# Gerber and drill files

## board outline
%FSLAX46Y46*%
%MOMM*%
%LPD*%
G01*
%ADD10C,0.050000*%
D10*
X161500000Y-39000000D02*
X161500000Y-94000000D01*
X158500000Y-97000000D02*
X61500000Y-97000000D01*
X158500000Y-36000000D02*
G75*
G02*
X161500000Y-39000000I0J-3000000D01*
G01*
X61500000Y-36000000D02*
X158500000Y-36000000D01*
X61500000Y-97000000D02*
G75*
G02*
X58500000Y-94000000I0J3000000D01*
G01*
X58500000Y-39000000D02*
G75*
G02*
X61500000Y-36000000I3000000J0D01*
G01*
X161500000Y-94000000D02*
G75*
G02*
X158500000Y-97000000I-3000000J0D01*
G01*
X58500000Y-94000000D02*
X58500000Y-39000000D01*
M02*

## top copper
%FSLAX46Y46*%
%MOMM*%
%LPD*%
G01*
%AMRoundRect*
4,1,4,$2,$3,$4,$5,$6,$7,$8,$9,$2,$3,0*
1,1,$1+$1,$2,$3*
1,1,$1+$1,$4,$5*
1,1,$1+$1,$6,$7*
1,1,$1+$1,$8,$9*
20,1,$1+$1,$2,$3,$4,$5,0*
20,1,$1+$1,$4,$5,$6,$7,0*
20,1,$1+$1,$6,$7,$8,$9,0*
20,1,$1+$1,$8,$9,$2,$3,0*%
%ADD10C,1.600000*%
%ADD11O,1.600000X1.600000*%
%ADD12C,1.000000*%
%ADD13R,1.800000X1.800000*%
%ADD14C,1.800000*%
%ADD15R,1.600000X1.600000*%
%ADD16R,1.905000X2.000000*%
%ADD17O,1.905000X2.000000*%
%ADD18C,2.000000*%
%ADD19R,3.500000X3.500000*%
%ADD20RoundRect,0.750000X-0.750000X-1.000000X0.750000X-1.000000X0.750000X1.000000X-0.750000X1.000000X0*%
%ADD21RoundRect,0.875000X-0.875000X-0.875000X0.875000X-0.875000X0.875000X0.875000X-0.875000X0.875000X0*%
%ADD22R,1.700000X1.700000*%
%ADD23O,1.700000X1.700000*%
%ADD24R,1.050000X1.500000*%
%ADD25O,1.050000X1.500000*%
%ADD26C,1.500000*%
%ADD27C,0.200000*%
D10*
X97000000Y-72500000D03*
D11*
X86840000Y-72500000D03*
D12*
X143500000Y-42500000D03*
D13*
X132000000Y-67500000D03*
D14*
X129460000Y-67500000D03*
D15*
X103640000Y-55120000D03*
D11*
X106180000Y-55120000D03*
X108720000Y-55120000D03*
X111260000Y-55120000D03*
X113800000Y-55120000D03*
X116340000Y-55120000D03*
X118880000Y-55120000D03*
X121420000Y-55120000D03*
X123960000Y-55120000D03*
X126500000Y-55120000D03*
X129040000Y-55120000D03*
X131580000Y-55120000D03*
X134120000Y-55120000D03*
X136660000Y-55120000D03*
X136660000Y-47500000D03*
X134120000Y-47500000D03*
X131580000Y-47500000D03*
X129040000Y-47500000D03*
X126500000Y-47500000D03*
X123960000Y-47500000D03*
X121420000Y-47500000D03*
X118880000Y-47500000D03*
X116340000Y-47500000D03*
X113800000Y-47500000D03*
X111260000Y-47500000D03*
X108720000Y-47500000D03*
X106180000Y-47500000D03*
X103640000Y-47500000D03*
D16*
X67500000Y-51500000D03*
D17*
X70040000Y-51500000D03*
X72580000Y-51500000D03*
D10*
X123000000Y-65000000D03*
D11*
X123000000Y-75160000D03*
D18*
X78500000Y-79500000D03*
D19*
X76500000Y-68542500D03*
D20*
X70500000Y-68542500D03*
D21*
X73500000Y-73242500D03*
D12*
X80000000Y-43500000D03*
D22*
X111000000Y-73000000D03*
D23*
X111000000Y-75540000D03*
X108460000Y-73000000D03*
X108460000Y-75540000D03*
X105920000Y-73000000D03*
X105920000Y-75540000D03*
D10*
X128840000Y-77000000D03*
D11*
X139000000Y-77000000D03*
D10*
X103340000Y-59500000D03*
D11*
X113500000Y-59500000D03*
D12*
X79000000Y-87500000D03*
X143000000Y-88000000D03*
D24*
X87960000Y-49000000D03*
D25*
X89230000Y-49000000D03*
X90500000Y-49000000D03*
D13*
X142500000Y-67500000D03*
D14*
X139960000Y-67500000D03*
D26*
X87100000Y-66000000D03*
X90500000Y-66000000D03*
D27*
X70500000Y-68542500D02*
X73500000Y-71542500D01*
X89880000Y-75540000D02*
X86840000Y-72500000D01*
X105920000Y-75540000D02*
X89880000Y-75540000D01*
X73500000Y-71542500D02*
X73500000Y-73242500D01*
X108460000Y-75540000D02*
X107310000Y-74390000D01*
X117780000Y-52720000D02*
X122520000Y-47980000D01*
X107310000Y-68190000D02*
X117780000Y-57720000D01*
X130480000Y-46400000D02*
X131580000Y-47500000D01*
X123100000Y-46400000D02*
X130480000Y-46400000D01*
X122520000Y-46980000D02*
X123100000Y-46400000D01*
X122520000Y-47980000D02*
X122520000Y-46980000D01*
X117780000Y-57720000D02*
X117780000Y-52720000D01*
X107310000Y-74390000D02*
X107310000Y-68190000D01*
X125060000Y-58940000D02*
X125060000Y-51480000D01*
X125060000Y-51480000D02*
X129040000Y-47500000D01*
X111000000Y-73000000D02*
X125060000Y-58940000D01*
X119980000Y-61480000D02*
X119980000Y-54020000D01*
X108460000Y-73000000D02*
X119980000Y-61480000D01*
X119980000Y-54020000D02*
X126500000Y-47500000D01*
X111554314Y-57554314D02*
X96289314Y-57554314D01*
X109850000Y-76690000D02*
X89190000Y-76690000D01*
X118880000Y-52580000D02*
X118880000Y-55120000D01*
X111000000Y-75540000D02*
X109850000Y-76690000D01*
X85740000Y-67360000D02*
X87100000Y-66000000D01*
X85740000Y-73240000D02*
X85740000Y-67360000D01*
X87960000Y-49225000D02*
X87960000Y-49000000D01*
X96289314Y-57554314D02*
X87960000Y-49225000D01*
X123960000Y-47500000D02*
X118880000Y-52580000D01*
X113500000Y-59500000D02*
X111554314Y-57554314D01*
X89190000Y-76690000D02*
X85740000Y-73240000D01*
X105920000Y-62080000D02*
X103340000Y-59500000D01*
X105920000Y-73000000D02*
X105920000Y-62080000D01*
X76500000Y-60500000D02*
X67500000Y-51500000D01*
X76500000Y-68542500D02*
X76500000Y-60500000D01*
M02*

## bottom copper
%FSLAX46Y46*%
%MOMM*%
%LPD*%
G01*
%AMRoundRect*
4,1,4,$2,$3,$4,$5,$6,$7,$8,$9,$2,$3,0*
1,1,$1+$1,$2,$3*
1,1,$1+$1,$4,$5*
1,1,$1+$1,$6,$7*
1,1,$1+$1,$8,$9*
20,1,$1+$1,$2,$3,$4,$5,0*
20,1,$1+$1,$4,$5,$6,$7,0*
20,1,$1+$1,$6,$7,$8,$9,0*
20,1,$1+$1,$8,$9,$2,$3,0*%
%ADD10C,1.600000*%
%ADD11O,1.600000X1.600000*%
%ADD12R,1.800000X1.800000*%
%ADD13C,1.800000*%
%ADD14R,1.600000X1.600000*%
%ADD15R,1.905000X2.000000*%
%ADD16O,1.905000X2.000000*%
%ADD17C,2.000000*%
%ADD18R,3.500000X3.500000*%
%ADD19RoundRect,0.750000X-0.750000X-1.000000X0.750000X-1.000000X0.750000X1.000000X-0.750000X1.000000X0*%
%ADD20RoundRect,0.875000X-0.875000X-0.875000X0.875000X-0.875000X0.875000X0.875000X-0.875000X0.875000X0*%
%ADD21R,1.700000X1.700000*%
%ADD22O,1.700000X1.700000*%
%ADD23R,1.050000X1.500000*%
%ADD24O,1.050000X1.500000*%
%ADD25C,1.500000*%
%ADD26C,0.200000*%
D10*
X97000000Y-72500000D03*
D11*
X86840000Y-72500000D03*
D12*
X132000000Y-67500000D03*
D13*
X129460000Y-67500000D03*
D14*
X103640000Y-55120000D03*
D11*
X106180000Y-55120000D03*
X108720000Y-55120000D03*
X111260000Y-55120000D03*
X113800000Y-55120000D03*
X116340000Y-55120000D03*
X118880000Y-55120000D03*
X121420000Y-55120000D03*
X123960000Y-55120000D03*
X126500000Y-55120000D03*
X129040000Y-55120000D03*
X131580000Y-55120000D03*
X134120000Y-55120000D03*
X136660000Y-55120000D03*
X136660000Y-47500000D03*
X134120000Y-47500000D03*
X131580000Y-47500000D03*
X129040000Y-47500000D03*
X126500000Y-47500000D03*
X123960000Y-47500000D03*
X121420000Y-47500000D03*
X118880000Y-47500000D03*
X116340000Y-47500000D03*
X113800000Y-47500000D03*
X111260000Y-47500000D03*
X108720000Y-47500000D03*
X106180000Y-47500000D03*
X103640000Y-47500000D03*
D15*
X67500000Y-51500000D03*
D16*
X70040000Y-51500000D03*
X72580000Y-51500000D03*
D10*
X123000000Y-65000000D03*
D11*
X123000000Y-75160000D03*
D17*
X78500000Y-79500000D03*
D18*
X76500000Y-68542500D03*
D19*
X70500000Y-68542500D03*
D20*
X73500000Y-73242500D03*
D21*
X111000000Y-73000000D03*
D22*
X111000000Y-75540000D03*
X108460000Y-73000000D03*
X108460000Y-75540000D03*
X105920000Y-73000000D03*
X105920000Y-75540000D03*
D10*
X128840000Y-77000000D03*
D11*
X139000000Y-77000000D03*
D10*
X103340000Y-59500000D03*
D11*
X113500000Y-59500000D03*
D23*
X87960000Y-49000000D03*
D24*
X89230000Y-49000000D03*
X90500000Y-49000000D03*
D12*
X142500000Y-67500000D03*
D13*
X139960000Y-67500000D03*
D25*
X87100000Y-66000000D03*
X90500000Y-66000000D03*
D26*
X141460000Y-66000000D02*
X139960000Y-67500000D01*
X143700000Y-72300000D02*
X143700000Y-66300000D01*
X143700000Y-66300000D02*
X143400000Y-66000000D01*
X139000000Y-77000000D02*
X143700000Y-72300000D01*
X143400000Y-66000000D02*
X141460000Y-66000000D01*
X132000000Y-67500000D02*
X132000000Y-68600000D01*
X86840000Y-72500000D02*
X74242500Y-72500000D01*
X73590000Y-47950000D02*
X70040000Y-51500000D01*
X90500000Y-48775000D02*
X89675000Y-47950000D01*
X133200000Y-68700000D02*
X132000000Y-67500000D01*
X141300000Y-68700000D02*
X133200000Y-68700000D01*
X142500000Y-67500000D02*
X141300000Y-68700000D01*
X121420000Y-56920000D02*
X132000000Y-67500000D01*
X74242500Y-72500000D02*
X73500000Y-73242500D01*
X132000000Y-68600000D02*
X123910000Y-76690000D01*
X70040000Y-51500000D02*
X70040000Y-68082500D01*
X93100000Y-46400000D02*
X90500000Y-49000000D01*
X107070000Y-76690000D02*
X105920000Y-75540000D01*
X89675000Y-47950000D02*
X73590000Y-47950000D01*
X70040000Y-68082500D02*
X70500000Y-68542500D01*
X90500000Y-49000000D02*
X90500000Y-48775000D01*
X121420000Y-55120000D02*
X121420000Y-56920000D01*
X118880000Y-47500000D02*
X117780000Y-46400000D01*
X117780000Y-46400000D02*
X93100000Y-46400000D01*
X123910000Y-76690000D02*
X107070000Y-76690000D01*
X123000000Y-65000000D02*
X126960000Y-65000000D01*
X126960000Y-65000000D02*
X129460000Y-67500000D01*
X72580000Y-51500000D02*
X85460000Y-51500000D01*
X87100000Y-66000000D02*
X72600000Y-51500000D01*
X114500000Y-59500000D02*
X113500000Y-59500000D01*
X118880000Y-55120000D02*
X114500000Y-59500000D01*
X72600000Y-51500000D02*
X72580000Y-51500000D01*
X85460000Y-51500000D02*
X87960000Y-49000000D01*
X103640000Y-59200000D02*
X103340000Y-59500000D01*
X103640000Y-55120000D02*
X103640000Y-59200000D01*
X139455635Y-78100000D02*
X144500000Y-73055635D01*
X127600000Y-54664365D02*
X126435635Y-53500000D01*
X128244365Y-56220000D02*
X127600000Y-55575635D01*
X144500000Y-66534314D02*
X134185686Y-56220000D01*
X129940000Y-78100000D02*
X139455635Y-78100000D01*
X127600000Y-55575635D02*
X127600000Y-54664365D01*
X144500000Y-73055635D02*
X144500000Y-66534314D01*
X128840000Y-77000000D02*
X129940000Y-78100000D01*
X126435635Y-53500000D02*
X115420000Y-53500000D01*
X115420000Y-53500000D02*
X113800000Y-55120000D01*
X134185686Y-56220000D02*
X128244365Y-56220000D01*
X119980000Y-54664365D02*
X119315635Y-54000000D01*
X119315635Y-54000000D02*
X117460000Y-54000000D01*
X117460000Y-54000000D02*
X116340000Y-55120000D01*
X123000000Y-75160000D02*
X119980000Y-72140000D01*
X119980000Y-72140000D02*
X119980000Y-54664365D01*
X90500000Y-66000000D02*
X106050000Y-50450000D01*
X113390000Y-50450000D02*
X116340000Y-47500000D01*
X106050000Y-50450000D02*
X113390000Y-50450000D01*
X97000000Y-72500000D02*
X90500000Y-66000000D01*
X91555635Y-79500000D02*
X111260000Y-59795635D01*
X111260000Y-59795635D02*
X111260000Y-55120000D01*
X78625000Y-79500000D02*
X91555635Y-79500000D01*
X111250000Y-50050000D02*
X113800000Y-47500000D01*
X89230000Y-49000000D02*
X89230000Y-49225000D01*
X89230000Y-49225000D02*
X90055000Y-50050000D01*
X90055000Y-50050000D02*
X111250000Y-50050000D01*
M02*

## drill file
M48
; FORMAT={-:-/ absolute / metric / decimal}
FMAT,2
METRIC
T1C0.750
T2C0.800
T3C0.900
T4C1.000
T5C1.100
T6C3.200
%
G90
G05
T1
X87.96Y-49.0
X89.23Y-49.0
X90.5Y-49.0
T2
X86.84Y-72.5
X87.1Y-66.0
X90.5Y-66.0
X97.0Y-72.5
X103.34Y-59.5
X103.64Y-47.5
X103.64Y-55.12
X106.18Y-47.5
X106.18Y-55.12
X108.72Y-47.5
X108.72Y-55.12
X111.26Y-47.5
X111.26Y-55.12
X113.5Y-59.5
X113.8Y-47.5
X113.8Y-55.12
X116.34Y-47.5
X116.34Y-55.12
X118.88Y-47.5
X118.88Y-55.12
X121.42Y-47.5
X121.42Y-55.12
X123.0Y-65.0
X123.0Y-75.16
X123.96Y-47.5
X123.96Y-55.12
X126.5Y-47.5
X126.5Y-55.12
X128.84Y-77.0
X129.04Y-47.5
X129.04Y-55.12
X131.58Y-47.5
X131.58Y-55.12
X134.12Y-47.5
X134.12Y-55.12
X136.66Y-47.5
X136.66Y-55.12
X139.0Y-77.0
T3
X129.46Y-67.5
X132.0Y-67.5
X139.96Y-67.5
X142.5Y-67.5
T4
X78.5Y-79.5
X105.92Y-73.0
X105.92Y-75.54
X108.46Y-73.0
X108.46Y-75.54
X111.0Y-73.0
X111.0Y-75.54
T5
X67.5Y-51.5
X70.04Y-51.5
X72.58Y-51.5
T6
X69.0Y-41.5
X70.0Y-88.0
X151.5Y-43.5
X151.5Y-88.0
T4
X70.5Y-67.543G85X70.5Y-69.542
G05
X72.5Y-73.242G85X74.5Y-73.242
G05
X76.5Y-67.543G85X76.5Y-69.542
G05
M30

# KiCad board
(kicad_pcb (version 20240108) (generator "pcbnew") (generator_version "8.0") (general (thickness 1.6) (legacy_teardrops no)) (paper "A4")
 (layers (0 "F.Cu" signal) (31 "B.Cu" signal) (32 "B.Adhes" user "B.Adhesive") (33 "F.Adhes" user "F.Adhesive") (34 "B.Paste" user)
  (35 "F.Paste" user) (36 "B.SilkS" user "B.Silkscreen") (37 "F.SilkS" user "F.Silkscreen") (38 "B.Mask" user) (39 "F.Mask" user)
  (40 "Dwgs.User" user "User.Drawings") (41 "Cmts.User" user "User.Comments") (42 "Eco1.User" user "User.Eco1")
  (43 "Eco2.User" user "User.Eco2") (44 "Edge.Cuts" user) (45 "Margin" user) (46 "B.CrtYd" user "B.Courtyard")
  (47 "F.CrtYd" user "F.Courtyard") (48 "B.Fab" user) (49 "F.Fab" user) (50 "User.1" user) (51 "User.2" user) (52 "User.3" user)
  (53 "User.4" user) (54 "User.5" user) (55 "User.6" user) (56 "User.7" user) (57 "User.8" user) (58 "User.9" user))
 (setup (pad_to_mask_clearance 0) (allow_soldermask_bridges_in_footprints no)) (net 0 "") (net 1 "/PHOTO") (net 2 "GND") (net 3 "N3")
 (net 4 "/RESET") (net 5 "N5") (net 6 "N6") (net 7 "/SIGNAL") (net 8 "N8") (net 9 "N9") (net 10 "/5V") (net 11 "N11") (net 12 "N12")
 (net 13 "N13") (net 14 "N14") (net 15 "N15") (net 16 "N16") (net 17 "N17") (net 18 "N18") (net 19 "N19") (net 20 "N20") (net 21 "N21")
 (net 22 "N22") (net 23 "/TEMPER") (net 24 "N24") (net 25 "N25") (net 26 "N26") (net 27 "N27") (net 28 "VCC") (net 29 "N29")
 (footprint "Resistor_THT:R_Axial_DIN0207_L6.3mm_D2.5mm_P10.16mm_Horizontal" (layer "F.Cu") (at 97 72.5 180)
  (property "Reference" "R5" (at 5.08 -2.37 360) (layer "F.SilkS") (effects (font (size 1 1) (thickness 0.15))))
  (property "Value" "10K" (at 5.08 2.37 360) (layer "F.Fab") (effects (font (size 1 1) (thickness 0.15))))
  (pad "1" thru_hole circle (at 0 0 180) (size 1.6 1.6) (drill 0.8) (layers "*.Cu" "*.Mask") (remove_unused_layers no) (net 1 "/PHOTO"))
  (pad "2" thru_hole oval (at 10.16 0 180) (size 1.6 1.6) (drill 0.8) (layers "*.Cu" "*.Mask") (remove_unused_layers no) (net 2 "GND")))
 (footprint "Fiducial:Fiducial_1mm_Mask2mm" (layer "F.Cu") (at 143.5 42.5)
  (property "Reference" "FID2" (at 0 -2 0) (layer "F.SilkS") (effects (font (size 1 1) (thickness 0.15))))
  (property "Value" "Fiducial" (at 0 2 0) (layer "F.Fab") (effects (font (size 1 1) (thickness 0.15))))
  (pad "" smd circle (at 0 0) (size 1 1) (layers "F.Cu" "F.Mask") (solder_mask_margin 0.5) (clearance 0.5)))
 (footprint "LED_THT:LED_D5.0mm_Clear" (layer "F.Cu") (at 132 67.5 180)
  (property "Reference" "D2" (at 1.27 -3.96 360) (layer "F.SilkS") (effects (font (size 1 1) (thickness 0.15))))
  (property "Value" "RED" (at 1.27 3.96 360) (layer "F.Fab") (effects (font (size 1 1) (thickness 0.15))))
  (pad "1" thru_hole rect (at 0 0 180) (size 1.8 1.8) (drill 0.9) (layers "*.Cu" "*.Mask") (remove_unused_layers no) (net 2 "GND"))
  (pad "2" thru_hole circle (at 2.54 0 180) (size 1.8 1.8) (drill 0.9) (layers "*.Cu" "*.Mask") (remove_unused_layers no) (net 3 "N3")))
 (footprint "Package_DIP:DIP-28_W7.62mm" (layer "F.Cu") (at 103.64 55.12 90)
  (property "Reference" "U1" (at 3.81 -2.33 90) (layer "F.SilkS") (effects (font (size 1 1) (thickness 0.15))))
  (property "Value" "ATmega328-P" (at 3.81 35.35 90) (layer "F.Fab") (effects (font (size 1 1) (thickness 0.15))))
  (pad "1" thru_hole rect (at 0 0 90) (size 1.6 1.6) (drill 0.8) (layers "*.Cu" "*.Mask") (remove_unused_layers no) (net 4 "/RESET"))
  (pad "2" thru_hole oval (at 0 2.54 90) (size 1.6 1.6) (drill 0.8) (layers "*.Cu" "*.Mask") (remove_unused_layers no) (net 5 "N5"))
  (pad "3" thru_hole oval (at 0 5.08 90) (size 1.6 1.6) (drill 0.8) (layers "*.Cu" "*.Mask") (remove_unused_layers no) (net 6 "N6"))
  (pad "4" thru_hole oval (at 0 7.62 90) (size 1.6 1.6) (drill 0.8) (layers "*.Cu" "*.Mask") (remove_unused_layers no) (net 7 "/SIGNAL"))
  (pad "5" thru_hole oval (at 0 10.16 90) (size 1.6 1.6) (drill 0.8) (layers "*.Cu" "*.Mask") (remove_unused_layers no) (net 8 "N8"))
  (pad "6" thru_hole oval (at 0 12.7 90) (size 1.6 1.6) (drill 0.8) (layers "*.Cu" "*.Mask") (remove_unused_layers no) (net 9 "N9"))
  (pad "7" thru_hole oval (at 0 15.24 90) (size 1.6 1.6) (drill 0.8) (layers "*.Cu" "*.Mask") (remove_unused_layers no) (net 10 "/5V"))
  (pad "8" thru_hole oval (at 0 17.78 90) (size 1.6 1.6) (drill 0.8) (layers "*.Cu" "*.Mask") (remove_unused_layers no) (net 2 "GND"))
  (pad "9" thru_hole oval (at 0 20.32 90) (size 1.6 1.6) (drill 0.8) (layers "*.Cu" "*.Mask") (remove_unused_layers no) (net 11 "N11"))
  (pad "10" thru_hole oval (at 0 22.86 90) (size 1.6 1.6) (drill 0.8) (layers "*.Cu" "*.Mask") (remove_unused_layers no) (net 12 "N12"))
  (pad "11" thru_hole oval (at 0 25.4 90) (size 1.6 1.6) (drill 0.8) (layers "*.Cu" "*.Mask") (remove_unused_layers no) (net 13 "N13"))
  (pad "12" thru_hole oval (at 0 27.94 90) (size 1.6 1.6) (drill 0.8) (layers "*.Cu" "*.Mask") (remove_unused_layers no) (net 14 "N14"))
  (pad "13" thru_hole oval (at 0 30.48 90) (size 1.6 1.6) (drill 0.8) (layers "*.Cu" "*.Mask") (remove_unused_layers no) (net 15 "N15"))
  (pad "14" thru_hole oval (at 0 33.02 90) (size 1.6 1.6) (drill 0.8) (layers "*.Cu" "*.Mask") (remove_unused_layers no) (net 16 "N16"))
  (pad "15" thru_hole oval (at 7.62 33.02 90) (size 1.6 1.6) (drill 0.8) (layers "*.Cu" "*.Mask") (remove_unused_layers no) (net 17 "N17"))
  (pad "16" thru_hole oval (at 7.62 30.48 90) (size 1.6 1.6) (drill 0.8) (layers "*.Cu" "*.Mask") (remove_unused_layers no) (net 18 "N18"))
  (pad "17" thru_hole oval (at 7.62 27.94 90) (size 1.6 1.6) (drill 0.8) (layers "*.Cu" "*.Mask") (remove_unused_layers no) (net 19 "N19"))
  (pad "18" thru_hole oval (at 7.62 25.4 90) (size 1.6 1.6) (drill 0.8) (layers "*.Cu" "*.Mask") (remove_unused_layers no) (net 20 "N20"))
  (pad "19" thru_hole oval (at 7.62 22.86 90) (size 1.6 1.6) (drill 0.8) (layers "*.Cu" "*.Mask") (remove_unused_layers no) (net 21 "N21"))
  (pad "20" thru_hole oval (at 7.62 20.32 90) (size 1.6 1.6) (drill 0.8) (layers "*.Cu" "*.Mask") (remove_unused_layers no) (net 10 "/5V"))
  (pad "21" thru_hole oval (at 7.62 17.78 90) (size 1.6 1.6) (drill 0.8) (layers "*.Cu" "*.Mask") (remove_unused_layers no) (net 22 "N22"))
  (pad "22" thru_hole oval (at 7.62 15.24 90) (size 1.6 1.6) (drill 0.8) (layers "*.Cu" "*.Mask") (remove_unused_layers no) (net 2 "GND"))
  (pad "23" thru_hole oval (at 7.62 12.7 90) (size 1.6 1.6) (drill 0.8) (layers "*.Cu" "*.Mask") (remove_unused_layers no) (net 1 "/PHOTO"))
  (pad "24" thru_hole oval (at 7.62 10.16 90) (size 1.6 1.6) (drill 0.8) (layers "*.Cu" "*.Mask") (remove_unused_layers no)
   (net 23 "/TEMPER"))
  (pad "25" thru_hole oval (at 7.62 7.62 90) (size 1.6 1.6) (drill 0.8) (layers "*.Cu" "*.Mask") (remove_unused_layers no) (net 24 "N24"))
  (pad "26" thru_hole oval (at 7.62 5.08 90) (size 1.6 1.6) (drill 0.8) (layers "*.Cu" "*.Mask") (remove_unused_layers no) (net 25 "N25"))
  (pad "27" thru_hole oval (at 7.62 2.54 90) (size 1.6 1.6) (drill 0.8) (layers "*.Cu" "*.Mask") (remove_unused_layers no) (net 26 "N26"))
  (pad "28" thru_hole oval (at 7.62 0 90) (size 1.6 1.6) (drill 0.8) (layers "*.Cu" "*.Mask") (remove_unused_layers no) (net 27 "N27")))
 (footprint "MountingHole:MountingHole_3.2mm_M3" (layer "F.Cu") (at 151.5 88)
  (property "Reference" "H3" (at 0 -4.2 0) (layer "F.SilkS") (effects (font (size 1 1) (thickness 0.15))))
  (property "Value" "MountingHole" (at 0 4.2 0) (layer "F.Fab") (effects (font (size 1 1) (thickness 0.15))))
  (pad "" np_thru_hole circle (at 0 0) (size 3.2 3.2) (drill 3.2) (layers "*.Cu" "*.Mask")))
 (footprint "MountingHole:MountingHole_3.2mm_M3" (layer "F.Cu") (at 151.5 43.5)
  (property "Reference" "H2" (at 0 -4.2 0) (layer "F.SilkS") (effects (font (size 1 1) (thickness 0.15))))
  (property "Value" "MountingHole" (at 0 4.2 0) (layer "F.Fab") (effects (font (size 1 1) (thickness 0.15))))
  (pad "" np_thru_hole circle (at 0 0) (size 3.2 3.2) (drill 3.2) (layers "*.Cu" "*.Mask")))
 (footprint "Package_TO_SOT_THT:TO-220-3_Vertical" (layer "F.Cu") (at 67.5 51.5)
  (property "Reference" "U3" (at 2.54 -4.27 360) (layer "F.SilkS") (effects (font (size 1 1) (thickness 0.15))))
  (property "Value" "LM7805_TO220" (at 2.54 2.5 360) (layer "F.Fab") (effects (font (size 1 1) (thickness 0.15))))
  (pad "1" thru_hole rect (at 0 0) (size 1.905 2) (drill 1.1) (layers "*.Cu" "*.Mask") (remove_unused_layers no) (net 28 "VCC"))
  (pad "2" thru_hole oval (at 2.54 0) (size 1.905 2) (drill 1.1) (layers "*.Cu" "*.Mask") (remove_unused_layers no) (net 2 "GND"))
  (pad "3" thru_hole oval (at 5.08 0) (size 1.905 2) (drill 1.1) (layers "*.Cu" "*.Mask") (remove_unused_layers no) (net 10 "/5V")))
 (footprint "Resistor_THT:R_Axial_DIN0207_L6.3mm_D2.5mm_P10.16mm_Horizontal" (layer "F.Cu") (at 123 65 -90)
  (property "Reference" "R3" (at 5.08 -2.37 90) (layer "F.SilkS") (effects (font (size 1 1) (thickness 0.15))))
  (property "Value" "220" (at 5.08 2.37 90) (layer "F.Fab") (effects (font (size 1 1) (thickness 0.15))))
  (pad "1" thru_hole circle (at 0 0 270) (size 1.6 1.6) (drill 0.8) (layers "*.Cu" "*.Mask") (remove_unused_layers no) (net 3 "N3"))
  (pad "2" thru_hole oval (at 10.16 0 270) (size 1.6 1.6) (drill 0.8) (layers "*.Cu" "*.Mask") (remove_unused_layers no) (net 9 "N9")))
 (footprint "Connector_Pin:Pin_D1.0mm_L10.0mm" (layer "F.Cu") (at 78.5 79.5)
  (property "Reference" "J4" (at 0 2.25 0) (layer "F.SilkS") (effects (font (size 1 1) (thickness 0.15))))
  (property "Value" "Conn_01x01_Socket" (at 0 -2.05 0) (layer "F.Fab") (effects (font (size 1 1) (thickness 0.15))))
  (pad "1" thru_hole circle (at 0 0) (size 2 2) (drill 1) (layers "*.Cu" "*.Mask") (remove_unused_layers no) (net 7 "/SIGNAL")))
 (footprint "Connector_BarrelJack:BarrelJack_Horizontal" (layer "F.Cu") (at 76.5 68.5425)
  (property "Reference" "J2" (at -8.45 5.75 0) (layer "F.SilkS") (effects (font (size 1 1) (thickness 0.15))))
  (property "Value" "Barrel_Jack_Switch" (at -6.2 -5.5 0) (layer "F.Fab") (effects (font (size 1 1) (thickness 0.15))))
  (pad "1" thru_hole rect (at 0 0) (size 3.5 3.5) (drill oval 1 3) (layers "*.Cu" "*.Mask") (remove_unused_layers no) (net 28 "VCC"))
  (pad "2" thru_hole roundrect (at -6 0) (size 3 3.5) (drill oval 1 3) (layers "*.Cu" "*.Mask") (remove_unused_layers no)
   (roundrect_rratio 0.25) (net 2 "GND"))
  (pad "3" thru_hole roundrect (at -3 4.7) (size 3.5 3.5) (drill oval 3 1) (layers "*.Cu" "*.Mask") (remove_unused_layers no)
   (roundrect_rratio 0.25) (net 2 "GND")))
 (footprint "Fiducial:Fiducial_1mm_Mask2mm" (layer "F.Cu") (at 80 43.5)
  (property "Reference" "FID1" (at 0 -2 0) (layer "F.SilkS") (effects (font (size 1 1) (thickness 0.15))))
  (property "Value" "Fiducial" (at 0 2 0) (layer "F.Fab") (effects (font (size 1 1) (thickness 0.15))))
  (pad "" smd circle (at 0 0) (size 1 1) (layers "F.Cu" "F.Mask") (solder_mask_margin 0.5) (clearance 0.5)))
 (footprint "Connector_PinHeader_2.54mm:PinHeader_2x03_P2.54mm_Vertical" (layer "F.Cu") (at 111 73 -90)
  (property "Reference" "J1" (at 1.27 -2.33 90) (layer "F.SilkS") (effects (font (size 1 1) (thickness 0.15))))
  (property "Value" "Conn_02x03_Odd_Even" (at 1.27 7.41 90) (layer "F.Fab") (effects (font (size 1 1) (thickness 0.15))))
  (pad "1" thru_hole rect (at 0 0 270) (size 1.7 1.7) (drill 1) (layers "*.Cu" "*.Mask") (remove_unused_layers no) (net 20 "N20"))
  (pad "2" thru_hole oval (at 2.54 0 270) (size 1.7 1.7) (drill 1) (layers "*.Cu" "*.Mask") (remove_unused_layers no) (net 10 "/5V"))
  (pad "3" thru_hole oval (at 0 2.54 270) (size 1.7 1.7) (drill 1) (layers "*.Cu" "*.Mask") (remove_unused_layers no) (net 21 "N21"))
  (pad "4" thru_hole oval (at 2.54 2.54 270) (size 1.7 1.7) (drill 1) (layers "*.Cu" "*.Mask") (remove_unused_layers no) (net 19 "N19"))
  (pad "5" thru_hole oval (at 0 5.08 270) (size 1.7 1.7) (drill 1) (layers "*.Cu" "*.Mask") (remove_unused_layers no) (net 4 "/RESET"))
  (pad "6" thru_hole oval (at 2.54 5.08 270) (size 1.7 1.7) (drill 1) (layers "*.Cu" "*.Mask") (remove_unused_layers no) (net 2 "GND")))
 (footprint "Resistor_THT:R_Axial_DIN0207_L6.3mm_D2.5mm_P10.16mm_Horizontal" (layer "F.Cu") (at 128.84 77)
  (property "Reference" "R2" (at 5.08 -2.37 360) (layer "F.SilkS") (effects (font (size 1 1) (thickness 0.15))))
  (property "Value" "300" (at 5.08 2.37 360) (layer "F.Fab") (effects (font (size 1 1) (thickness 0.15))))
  (pad "1" thru_hole circle (at 0 0) (size 1.6 1.6) (drill 0.8) (layers "*.Cu" "*.Mask") (remove_unused_layers no) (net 8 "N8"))
  (pad "2" thru_hole oval (at 10.16 0) (size 1.6 1.6) (drill 0.8) (layers "*.Cu" "*.Mask") (remove_unused_layers no) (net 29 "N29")))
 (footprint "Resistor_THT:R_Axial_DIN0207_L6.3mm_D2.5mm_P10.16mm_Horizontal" (layer "F.Cu") (at 103.34 59.5)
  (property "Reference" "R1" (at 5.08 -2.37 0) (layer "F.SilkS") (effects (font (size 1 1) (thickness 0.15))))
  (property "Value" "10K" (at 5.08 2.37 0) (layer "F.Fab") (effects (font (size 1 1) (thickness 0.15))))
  (pad "1" thru_hole circle (at 0 0) (size 1.6 1.6) (drill 0.8) (layers "*.Cu" "*.Mask") (remove_unused_layers no) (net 4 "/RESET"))
  (pad "2" thru_hole oval (at 10.16 0) (size 1.6 1.6) (drill 0.8) (layers "*.Cu" "*.Mask") (remove_unused_layers no) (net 10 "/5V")))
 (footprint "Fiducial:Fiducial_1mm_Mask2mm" (layer "F.Cu") (at 79 87.5)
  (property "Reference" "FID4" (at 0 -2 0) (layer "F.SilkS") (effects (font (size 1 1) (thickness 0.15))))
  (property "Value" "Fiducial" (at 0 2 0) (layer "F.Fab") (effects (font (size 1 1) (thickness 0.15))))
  (pad "" smd circle (at 0 0) (size 1 1) (layers "F.Cu" "F.Mask") (solder_mask_margin 0.5) (clearance 0.5)))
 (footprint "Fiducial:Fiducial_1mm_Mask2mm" (layer "F.Cu") (at 143 88)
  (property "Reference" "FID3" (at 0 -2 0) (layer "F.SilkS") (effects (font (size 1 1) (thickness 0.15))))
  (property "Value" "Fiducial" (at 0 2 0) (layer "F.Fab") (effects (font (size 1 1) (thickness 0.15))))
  (pad "" smd circle (at 0 0) (size 1 1) (layers "F.Cu" "F.Mask") (solder_mask_margin 0.5) (clearance 0.5)))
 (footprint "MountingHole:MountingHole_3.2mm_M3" (layer "F.Cu") (at 69 41.5)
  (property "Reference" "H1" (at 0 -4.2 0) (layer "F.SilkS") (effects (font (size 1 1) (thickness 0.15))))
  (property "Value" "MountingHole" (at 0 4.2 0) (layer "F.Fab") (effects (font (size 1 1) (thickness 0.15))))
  (pad "" np_thru_hole circle (at 0 0) (size 3.2 3.2) (drill 3.2) (layers "*.Cu" "*.Mask")))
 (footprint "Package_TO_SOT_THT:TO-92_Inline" (layer "F.Cu") (at 87.96 49)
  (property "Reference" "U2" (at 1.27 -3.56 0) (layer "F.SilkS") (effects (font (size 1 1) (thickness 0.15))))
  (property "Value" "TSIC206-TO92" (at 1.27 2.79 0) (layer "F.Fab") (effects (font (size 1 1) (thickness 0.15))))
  (pad "1" thru_hole rect (at 0 0) (size 1.05 1.5) (drill 0.75) (layers "*.Cu" "*.Mask") (remove_unused_layers no) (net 10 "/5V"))
  (pad "2" thru_hole oval (at 1.27 0) (size 1.05 1.5) (drill 0.75) (layers "*.Cu" "*.Mask") (remove_unused_layers no) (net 23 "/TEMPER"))
  (pad "3" thru_hole oval (at 2.54 0) (size 1.05 1.5) (drill 0.75) (layers "*.Cu" "*.Mask") (remove_unused_layers no) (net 2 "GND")))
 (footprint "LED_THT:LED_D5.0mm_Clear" (layer "F.Cu") (at 142.5 67.5 180)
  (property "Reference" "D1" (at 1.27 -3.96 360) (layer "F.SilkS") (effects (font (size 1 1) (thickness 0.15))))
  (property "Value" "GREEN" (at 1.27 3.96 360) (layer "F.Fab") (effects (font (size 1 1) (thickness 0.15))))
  (pad "1" thru_hole rect (at 0 0 180) (size 1.8 1.8) (drill 0.9) (layers "*.Cu" "*.Mask") (remove_unused_layers no) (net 2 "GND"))
  (pad "2" thru_hole circle (at 2.54 0 180) (size 1.8 1.8) (drill 0.9) (layers "*.Cu" "*.Mask") (remove_unused_layers no) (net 29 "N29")))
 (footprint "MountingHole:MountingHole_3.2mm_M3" (layer "F.Cu") (at 70 88)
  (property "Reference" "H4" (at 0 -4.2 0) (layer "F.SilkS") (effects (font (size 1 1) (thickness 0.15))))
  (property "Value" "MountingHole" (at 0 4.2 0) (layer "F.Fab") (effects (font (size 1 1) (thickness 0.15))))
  (pad "" np_thru_hole circle (at 0 0) (size 3.2 3.2) (drill 3.2) (layers "*.Cu" "*.Mask")))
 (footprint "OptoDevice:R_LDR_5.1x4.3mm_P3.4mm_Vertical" (layer "F.Cu") (at 87.1 66)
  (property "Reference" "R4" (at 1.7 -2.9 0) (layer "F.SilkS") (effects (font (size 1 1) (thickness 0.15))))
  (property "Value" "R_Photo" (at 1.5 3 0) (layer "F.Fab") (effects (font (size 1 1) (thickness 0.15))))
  (pad "1" thru_hole circle (at 0 0) (size 1.5 1.5) (drill 0.8) (layers "*.Cu" "*.Mask") (remove_unused_layers no) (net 10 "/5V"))
  (pad "2" thru_hole circle (at 3.4 0) (size 1.5 1.5) (drill 0.8) (layers "*.Cu" "*.Mask") (remove_unused_layers no) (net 1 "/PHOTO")))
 (gr_line (start 161.5 39) (end 161.5 94) (stroke (width 0.05) (type default)) (layer "Edge.Cuts"))
 (gr_line (start 158.5 97) (end 61.5 97) (stroke (width 0.05) (type default)) (layer "Edge.Cuts"))
 (gr_arc (start 158.5 36) (mid 160.62132 36.87868) (end 161.5 39) (stroke (width 0.05) (type default)) (layer "Edge.Cuts"))
 (gr_line (start 61.5 36) (end 158.5 36) (stroke (width 0.05) (type default)) (layer "Edge.Cuts"))
 (gr_arc (start 61.5 97) (mid 59.37868 96.12132) (end 58.5 94) (stroke (width 0.05) (type default)) (layer "Edge.Cuts"))
 (gr_arc (start 58.5 39) (mid 59.37868 36.87868) (end 61.5 36) (stroke (width 0.05) (type default)) (layer "Edge.Cuts"))
 (gr_arc (start 161.5 94) (mid 160.62132 96.12132) (end 158.5 97) (stroke (width 0.05) (type default)) (layer "Edge.Cuts"))
 (gr_line (start 58.5 94) (end 58.5 39) (stroke (width 0.05) (type default)) (layer "Edge.Cuts"))
 (segment (start 141.46 66) (end 139.96 67.5) (width 0.2) (layer "B.Cu") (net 29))
 (segment (start 143.7 72.3) (end 143.7 66.3) (width 0.2) (layer "B.Cu") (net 29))
 (segment (start 143.7 66.3) (end 143.4 66) (width 0.2) (layer "B.Cu") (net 29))
 (segment (start 139 77) (end 143.7 72.3) (width 0.2) (layer "B.Cu") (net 29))
 (segment (start 143.4 66) (end 141.46 66) (width 0.2) (layer "B.Cu") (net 29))
 (segment (start 70.5 68.5425) (end 73.5 71.5425) (width 0.2) (layer "F.Cu") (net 2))
 (segment (start 89.88 75.54) (end 86.84 72.5) (width 0.2) (layer "F.Cu") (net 2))
 (segment (start 105.92 75.54) (end 89.88 75.54) (width 0.2) (layer "F.Cu") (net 2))
 (segment (start 73.5 71.5425) (end 73.5 73.2425) (width 0.2) (layer "F.Cu") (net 2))
 (segment (start 132 67.5) (end 132 68.6) (width 0.2) (layer "B.Cu") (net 2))
 (segment (start 86.84 72.5) (end 74.2425 72.5) (width 0.2) (layer "B.Cu") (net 2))
 (segment (start 73.59 47.95) (end 70.04 51.5) (width 0.2) (layer "B.Cu") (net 2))
 (segment (start 90.5 48.775) (end 89.675 47.95) (width 0.2) (layer "B.Cu") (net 2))
 (segment (start 133.2 68.7) (end 132 67.5) (width 0.2) (layer "B.Cu") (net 2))
 (segment (start 141.3 68.7) (end 133.2 68.7) (width 0.2) (layer "B.Cu") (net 2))
 (segment (start 142.5 67.5) (end 141.3 68.7) (width 0.2) (layer "B.Cu") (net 2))
 (segment (start 121.42 56.92) (end 132 67.5) (width 0.2) (layer "B.Cu") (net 2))
 (segment (start 74.2425 72.5) (end 73.5 73.2425) (width 0.2) (layer "B.Cu") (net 2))
 (segment (start 132 68.6) (end 123.91 76.69) (width 0.2) (layer "B.Cu") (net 2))
 (segment (start 70.04 51.5) (end 70.04 68.0825) (width 0.2) (layer "B.Cu") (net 2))
 (segment (start 93.1 46.4) (end 90.5 49) (width 0.2) (layer "B.Cu") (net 2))
 (segment (start 107.07 76.69) (end 105.92 75.54) (width 0.2) (layer "B.Cu") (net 2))
 (segment (start 89.675 47.95) (end 73.59 47.95) (width 0.2) (layer "B.Cu") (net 2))
 (segment (start 70.04 68.0825) (end 70.5 68.5425) (width 0.2) (layer "B.Cu") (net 2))
 (segment (start 90.5 49) (end 90.5 48.775) (width 0.2) (layer "B.Cu") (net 2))
 (segment (start 121.42 55.12) (end 121.42 56.92) (width 0.2) (layer "B.Cu") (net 2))
 (segment (start 118.88 47.5) (end 117.78 46.4) (width 0.2) (layer "B.Cu") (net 2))
 (segment (start 117.78 46.4) (end 93.1 46.4) (width 0.2) (layer "B.Cu") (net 2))
 (segment (start 123.91 76.69) (end 107.07 76.69) (width 0.2) (layer "B.Cu") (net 2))
 (segment (start 123 65) (end 126.96 65) (width 0.2) (layer "B.Cu") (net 3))
 (segment (start 126.96 65) (end 129.46 67.5) (width 0.2) (layer "B.Cu") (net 3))
 (segment (start 108.46 75.54) (end 107.31 74.39) (width 0.2) (layer "F.Cu") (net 19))
 (segment (start 117.78 52.72) (end 122.52 47.98) (width 0.2) (layer "F.Cu") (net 19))
 (segment (start 107.31 68.19) (end 117.78 57.72) (width 0.2) (layer "F.Cu") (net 19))
 (segment (start 130.48 46.4) (end 131.58 47.5) (width 0.2) (layer "F.Cu") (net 19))
 (segment (start 123.1 46.4) (end 130.48 46.4) (width 0.2) (layer "F.Cu") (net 19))
 (segment (start 122.52 46.98) (end 123.1 46.4) (width 0.2) (layer "F.Cu") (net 19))
 (segment (start 122.52 47.98) (end 122.52 46.98) (width 0.2) (layer "F.Cu") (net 19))
 (segment (start 117.78 57.72) (end 117.78 52.72) (width 0.2) (layer "F.Cu") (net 19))
 (segment (start 107.31 74.39) (end 107.31 68.19) (width 0.2) (layer "F.Cu") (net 19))
 (segment (start 125.06 58.94) (end 125.06 51.48) (width 0.2) (layer "F.Cu") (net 20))
 (segment (start 125.06 51.48) (end 129.04 47.5) (width 0.2) (layer "F.Cu") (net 20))
 (segment (start 111 73) (end 125.06 58.94) (width 0.2) (layer "F.Cu") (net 20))
 (segment (start 119.98 61.48) (end 119.98 54.02) (width 0.2) (layer "F.Cu") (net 21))
 (segment (start 108.46 73) (end 119.98 61.48) (width 0.2) (layer "F.Cu") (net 21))
 (segment (start 119.98 54.02) (end 126.5 47.5) (width 0.2) (layer "F.Cu") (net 21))
 (segment (start 111.554314 57.554314) (end 96.289314 57.554314) (width 0.2) (layer "F.Cu") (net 10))
 (segment (start 109.85 76.69) (end 89.19 76.69) (width 0.2) (layer "F.Cu") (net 10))
 (segment (start 118.88 52.58) (end 118.88 55.12) (width 0.2) (layer "F.Cu") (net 10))
 (segment (start 111 75.54) (end 109.85 76.69) (width 0.2) (layer "F.Cu") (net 10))
 (segment (start 85.74 67.36) (end 87.1 66) (width 0.2) (layer "F.Cu") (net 10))
 (segment (start 85.74 73.24) (end 85.74 67.36) (width 0.2) (layer "F.Cu") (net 10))
 (segment (start 87.96 49.225) (end 87.96 49) (width 0.2) (layer "F.Cu") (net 10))
 (segment (start 96.289314 57.554314) (end 87.96 49.225) (width 0.2) (layer "F.Cu") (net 10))
 (segment (start 123.96 47.5) (end 118.88 52.58) (width 0.2) (layer "F.Cu") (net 10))
 (segment (start 113.5 59.5) (end 111.554314 57.554314) (width 0.2) (layer "F.Cu") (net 10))
 (segment (start 89.19 76.69) (end 85.74 73.24) (width 0.2) (layer "F.Cu") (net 10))
 (segment (start 72.58 51.5) (end 85.46 51.5) (width 0.2) (layer "B.Cu") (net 10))
 (segment (start 87.1 66) (end 72.6 51.5) (width 0.2) (layer "B.Cu") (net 10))
 (segment (start 114.5 59.5) (end 113.5 59.5) (width 0.2) (layer "B.Cu") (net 10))
 (segment (start 118.88 55.12) (end 114.5 59.5) (width 0.2) (layer "B.Cu") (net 10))
 (segment (start 72.6 51.5) (end 72.58 51.5) (width 0.2) (layer "B.Cu") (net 10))
 (segment (start 85.46 51.5) (end 87.96 49) (width 0.2) (layer "B.Cu") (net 10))
 (segment (start 105.92 62.08) (end 103.34 59.5) (width 0.2) (layer "F.Cu") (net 4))
 (segment (start 105.92 73) (end 105.92 62.08) (width 0.2) (layer "F.Cu") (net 4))
 (segment (start 103.64 59.2) (end 103.34 59.5) (width 0.2) (layer "B.Cu") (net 4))
 (segment (start 103.64 55.12) (end 103.64 59.2) (width 0.2) (layer "B.Cu") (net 4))
 (segment (start 76.5 60.5) (end 67.5 51.5) (width 0.2) (layer "F.Cu") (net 28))
 (segment (start 76.5 68.5425) (end 76.5 60.5) (width 0.2) (layer "F.Cu") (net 28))
 (segment (start 139.455635 78.1) (end 144.5 73.055635) (width 0.2) (layer "B.Cu") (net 8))
 (segment (start 127.6 54.664365) (end 126.435635 53.5) (width 0.2) (layer "B.Cu") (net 8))
 (segment (start 128.244365 56.22) (end 127.6 55.575635) (width 0.2) (layer "B.Cu") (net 8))
 (segment (start 144.5 66.534314) (end 134.185686 56.22) (width 0.2) (layer "B.Cu") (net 8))
 (segment (start 129.94 78.1) (end 139.455635 78.1) (width 0.2) (layer "B.Cu") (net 8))
 (segment (start 127.6 55.575635) (end 127.6 54.664365) (width 0.2) (layer "B.Cu") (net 8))
 (segment (start 144.5 73.055635) (end 144.5 66.534314) (width 0.2) (layer "B.Cu") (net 8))
 (segment (start 128.84 77) (end 129.94 78.1) (width 0.2) (layer "B.Cu") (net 8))
 (segment (start 126.435635 53.5) (end 115.42 53.5) (width 0.2) (layer "B.Cu") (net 8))
 (segment (start 115.42 53.5) (end 113.8 55.12) (width 0.2) (layer "B.Cu") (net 8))
 (segment (start 134.185686 56.22) (end 128.244365 56.22) (width 0.2) (layer "B.Cu") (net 8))
 (segment (start 119.98 54.664365) (end 119.315635 54) (width 0.2) (layer "B.Cu") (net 9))
 (segment (start 119.315635 54) (end 117.46 54) (width 0.2) (layer "B.Cu") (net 9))
 (segment (start 117.46 54) (end 116.34 55.12) (width 0.2) (layer "B.Cu") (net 9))
 (segment (start 123 75.16) (end 119.98 72.14) (width 0.2) (layer "B.Cu") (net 9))
 (segment (start 119.98 72.14) (end 119.98 54.664365) (width 0.2) (layer "B.Cu") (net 9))
 (segment (start 90.5 66) (end 106.05 50.45) (width 0.2) (layer "B.Cu") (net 1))
 (segment (start 113.39 50.45) (end 116.34 47.5) (width 0.2) (layer "B.Cu") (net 1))
 (segment (start 106.05 50.45) (end 113.39 50.45) (width 0.2) (layer "B.Cu") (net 1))
 (segment (start 97 72.5) (end 90.5 66) (width 0.2) (layer "B.Cu") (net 1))
 (segment (start 91.555635 79.5) (end 111.26 59.795635) (width 0.2) (layer "B.Cu") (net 7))
 (segment (start 111.26 59.795635) (end 111.26 55.12) (width 0.2) (layer "B.Cu") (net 7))
 (segment (start 78.625 79.5) (end 91.555635 79.5) (width 0.2) (layer "B.Cu") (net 7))
 (segment (start 111.25 50.05) (end 113.8 47.5) (width 0.2) (layer "B.Cu") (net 23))
 (segment (start 89.23 49) (end 89.23 49.225) (width 0.2) (layer "B.Cu") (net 23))
 (segment (start 89.23 49.225) (end 90.055 50.05) (width 0.2) (layer "B.Cu") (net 23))
 (segment (start 90.055 50.05) (end 111.25 50.05) (width 0.2) (layer "B.Cu") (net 23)))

